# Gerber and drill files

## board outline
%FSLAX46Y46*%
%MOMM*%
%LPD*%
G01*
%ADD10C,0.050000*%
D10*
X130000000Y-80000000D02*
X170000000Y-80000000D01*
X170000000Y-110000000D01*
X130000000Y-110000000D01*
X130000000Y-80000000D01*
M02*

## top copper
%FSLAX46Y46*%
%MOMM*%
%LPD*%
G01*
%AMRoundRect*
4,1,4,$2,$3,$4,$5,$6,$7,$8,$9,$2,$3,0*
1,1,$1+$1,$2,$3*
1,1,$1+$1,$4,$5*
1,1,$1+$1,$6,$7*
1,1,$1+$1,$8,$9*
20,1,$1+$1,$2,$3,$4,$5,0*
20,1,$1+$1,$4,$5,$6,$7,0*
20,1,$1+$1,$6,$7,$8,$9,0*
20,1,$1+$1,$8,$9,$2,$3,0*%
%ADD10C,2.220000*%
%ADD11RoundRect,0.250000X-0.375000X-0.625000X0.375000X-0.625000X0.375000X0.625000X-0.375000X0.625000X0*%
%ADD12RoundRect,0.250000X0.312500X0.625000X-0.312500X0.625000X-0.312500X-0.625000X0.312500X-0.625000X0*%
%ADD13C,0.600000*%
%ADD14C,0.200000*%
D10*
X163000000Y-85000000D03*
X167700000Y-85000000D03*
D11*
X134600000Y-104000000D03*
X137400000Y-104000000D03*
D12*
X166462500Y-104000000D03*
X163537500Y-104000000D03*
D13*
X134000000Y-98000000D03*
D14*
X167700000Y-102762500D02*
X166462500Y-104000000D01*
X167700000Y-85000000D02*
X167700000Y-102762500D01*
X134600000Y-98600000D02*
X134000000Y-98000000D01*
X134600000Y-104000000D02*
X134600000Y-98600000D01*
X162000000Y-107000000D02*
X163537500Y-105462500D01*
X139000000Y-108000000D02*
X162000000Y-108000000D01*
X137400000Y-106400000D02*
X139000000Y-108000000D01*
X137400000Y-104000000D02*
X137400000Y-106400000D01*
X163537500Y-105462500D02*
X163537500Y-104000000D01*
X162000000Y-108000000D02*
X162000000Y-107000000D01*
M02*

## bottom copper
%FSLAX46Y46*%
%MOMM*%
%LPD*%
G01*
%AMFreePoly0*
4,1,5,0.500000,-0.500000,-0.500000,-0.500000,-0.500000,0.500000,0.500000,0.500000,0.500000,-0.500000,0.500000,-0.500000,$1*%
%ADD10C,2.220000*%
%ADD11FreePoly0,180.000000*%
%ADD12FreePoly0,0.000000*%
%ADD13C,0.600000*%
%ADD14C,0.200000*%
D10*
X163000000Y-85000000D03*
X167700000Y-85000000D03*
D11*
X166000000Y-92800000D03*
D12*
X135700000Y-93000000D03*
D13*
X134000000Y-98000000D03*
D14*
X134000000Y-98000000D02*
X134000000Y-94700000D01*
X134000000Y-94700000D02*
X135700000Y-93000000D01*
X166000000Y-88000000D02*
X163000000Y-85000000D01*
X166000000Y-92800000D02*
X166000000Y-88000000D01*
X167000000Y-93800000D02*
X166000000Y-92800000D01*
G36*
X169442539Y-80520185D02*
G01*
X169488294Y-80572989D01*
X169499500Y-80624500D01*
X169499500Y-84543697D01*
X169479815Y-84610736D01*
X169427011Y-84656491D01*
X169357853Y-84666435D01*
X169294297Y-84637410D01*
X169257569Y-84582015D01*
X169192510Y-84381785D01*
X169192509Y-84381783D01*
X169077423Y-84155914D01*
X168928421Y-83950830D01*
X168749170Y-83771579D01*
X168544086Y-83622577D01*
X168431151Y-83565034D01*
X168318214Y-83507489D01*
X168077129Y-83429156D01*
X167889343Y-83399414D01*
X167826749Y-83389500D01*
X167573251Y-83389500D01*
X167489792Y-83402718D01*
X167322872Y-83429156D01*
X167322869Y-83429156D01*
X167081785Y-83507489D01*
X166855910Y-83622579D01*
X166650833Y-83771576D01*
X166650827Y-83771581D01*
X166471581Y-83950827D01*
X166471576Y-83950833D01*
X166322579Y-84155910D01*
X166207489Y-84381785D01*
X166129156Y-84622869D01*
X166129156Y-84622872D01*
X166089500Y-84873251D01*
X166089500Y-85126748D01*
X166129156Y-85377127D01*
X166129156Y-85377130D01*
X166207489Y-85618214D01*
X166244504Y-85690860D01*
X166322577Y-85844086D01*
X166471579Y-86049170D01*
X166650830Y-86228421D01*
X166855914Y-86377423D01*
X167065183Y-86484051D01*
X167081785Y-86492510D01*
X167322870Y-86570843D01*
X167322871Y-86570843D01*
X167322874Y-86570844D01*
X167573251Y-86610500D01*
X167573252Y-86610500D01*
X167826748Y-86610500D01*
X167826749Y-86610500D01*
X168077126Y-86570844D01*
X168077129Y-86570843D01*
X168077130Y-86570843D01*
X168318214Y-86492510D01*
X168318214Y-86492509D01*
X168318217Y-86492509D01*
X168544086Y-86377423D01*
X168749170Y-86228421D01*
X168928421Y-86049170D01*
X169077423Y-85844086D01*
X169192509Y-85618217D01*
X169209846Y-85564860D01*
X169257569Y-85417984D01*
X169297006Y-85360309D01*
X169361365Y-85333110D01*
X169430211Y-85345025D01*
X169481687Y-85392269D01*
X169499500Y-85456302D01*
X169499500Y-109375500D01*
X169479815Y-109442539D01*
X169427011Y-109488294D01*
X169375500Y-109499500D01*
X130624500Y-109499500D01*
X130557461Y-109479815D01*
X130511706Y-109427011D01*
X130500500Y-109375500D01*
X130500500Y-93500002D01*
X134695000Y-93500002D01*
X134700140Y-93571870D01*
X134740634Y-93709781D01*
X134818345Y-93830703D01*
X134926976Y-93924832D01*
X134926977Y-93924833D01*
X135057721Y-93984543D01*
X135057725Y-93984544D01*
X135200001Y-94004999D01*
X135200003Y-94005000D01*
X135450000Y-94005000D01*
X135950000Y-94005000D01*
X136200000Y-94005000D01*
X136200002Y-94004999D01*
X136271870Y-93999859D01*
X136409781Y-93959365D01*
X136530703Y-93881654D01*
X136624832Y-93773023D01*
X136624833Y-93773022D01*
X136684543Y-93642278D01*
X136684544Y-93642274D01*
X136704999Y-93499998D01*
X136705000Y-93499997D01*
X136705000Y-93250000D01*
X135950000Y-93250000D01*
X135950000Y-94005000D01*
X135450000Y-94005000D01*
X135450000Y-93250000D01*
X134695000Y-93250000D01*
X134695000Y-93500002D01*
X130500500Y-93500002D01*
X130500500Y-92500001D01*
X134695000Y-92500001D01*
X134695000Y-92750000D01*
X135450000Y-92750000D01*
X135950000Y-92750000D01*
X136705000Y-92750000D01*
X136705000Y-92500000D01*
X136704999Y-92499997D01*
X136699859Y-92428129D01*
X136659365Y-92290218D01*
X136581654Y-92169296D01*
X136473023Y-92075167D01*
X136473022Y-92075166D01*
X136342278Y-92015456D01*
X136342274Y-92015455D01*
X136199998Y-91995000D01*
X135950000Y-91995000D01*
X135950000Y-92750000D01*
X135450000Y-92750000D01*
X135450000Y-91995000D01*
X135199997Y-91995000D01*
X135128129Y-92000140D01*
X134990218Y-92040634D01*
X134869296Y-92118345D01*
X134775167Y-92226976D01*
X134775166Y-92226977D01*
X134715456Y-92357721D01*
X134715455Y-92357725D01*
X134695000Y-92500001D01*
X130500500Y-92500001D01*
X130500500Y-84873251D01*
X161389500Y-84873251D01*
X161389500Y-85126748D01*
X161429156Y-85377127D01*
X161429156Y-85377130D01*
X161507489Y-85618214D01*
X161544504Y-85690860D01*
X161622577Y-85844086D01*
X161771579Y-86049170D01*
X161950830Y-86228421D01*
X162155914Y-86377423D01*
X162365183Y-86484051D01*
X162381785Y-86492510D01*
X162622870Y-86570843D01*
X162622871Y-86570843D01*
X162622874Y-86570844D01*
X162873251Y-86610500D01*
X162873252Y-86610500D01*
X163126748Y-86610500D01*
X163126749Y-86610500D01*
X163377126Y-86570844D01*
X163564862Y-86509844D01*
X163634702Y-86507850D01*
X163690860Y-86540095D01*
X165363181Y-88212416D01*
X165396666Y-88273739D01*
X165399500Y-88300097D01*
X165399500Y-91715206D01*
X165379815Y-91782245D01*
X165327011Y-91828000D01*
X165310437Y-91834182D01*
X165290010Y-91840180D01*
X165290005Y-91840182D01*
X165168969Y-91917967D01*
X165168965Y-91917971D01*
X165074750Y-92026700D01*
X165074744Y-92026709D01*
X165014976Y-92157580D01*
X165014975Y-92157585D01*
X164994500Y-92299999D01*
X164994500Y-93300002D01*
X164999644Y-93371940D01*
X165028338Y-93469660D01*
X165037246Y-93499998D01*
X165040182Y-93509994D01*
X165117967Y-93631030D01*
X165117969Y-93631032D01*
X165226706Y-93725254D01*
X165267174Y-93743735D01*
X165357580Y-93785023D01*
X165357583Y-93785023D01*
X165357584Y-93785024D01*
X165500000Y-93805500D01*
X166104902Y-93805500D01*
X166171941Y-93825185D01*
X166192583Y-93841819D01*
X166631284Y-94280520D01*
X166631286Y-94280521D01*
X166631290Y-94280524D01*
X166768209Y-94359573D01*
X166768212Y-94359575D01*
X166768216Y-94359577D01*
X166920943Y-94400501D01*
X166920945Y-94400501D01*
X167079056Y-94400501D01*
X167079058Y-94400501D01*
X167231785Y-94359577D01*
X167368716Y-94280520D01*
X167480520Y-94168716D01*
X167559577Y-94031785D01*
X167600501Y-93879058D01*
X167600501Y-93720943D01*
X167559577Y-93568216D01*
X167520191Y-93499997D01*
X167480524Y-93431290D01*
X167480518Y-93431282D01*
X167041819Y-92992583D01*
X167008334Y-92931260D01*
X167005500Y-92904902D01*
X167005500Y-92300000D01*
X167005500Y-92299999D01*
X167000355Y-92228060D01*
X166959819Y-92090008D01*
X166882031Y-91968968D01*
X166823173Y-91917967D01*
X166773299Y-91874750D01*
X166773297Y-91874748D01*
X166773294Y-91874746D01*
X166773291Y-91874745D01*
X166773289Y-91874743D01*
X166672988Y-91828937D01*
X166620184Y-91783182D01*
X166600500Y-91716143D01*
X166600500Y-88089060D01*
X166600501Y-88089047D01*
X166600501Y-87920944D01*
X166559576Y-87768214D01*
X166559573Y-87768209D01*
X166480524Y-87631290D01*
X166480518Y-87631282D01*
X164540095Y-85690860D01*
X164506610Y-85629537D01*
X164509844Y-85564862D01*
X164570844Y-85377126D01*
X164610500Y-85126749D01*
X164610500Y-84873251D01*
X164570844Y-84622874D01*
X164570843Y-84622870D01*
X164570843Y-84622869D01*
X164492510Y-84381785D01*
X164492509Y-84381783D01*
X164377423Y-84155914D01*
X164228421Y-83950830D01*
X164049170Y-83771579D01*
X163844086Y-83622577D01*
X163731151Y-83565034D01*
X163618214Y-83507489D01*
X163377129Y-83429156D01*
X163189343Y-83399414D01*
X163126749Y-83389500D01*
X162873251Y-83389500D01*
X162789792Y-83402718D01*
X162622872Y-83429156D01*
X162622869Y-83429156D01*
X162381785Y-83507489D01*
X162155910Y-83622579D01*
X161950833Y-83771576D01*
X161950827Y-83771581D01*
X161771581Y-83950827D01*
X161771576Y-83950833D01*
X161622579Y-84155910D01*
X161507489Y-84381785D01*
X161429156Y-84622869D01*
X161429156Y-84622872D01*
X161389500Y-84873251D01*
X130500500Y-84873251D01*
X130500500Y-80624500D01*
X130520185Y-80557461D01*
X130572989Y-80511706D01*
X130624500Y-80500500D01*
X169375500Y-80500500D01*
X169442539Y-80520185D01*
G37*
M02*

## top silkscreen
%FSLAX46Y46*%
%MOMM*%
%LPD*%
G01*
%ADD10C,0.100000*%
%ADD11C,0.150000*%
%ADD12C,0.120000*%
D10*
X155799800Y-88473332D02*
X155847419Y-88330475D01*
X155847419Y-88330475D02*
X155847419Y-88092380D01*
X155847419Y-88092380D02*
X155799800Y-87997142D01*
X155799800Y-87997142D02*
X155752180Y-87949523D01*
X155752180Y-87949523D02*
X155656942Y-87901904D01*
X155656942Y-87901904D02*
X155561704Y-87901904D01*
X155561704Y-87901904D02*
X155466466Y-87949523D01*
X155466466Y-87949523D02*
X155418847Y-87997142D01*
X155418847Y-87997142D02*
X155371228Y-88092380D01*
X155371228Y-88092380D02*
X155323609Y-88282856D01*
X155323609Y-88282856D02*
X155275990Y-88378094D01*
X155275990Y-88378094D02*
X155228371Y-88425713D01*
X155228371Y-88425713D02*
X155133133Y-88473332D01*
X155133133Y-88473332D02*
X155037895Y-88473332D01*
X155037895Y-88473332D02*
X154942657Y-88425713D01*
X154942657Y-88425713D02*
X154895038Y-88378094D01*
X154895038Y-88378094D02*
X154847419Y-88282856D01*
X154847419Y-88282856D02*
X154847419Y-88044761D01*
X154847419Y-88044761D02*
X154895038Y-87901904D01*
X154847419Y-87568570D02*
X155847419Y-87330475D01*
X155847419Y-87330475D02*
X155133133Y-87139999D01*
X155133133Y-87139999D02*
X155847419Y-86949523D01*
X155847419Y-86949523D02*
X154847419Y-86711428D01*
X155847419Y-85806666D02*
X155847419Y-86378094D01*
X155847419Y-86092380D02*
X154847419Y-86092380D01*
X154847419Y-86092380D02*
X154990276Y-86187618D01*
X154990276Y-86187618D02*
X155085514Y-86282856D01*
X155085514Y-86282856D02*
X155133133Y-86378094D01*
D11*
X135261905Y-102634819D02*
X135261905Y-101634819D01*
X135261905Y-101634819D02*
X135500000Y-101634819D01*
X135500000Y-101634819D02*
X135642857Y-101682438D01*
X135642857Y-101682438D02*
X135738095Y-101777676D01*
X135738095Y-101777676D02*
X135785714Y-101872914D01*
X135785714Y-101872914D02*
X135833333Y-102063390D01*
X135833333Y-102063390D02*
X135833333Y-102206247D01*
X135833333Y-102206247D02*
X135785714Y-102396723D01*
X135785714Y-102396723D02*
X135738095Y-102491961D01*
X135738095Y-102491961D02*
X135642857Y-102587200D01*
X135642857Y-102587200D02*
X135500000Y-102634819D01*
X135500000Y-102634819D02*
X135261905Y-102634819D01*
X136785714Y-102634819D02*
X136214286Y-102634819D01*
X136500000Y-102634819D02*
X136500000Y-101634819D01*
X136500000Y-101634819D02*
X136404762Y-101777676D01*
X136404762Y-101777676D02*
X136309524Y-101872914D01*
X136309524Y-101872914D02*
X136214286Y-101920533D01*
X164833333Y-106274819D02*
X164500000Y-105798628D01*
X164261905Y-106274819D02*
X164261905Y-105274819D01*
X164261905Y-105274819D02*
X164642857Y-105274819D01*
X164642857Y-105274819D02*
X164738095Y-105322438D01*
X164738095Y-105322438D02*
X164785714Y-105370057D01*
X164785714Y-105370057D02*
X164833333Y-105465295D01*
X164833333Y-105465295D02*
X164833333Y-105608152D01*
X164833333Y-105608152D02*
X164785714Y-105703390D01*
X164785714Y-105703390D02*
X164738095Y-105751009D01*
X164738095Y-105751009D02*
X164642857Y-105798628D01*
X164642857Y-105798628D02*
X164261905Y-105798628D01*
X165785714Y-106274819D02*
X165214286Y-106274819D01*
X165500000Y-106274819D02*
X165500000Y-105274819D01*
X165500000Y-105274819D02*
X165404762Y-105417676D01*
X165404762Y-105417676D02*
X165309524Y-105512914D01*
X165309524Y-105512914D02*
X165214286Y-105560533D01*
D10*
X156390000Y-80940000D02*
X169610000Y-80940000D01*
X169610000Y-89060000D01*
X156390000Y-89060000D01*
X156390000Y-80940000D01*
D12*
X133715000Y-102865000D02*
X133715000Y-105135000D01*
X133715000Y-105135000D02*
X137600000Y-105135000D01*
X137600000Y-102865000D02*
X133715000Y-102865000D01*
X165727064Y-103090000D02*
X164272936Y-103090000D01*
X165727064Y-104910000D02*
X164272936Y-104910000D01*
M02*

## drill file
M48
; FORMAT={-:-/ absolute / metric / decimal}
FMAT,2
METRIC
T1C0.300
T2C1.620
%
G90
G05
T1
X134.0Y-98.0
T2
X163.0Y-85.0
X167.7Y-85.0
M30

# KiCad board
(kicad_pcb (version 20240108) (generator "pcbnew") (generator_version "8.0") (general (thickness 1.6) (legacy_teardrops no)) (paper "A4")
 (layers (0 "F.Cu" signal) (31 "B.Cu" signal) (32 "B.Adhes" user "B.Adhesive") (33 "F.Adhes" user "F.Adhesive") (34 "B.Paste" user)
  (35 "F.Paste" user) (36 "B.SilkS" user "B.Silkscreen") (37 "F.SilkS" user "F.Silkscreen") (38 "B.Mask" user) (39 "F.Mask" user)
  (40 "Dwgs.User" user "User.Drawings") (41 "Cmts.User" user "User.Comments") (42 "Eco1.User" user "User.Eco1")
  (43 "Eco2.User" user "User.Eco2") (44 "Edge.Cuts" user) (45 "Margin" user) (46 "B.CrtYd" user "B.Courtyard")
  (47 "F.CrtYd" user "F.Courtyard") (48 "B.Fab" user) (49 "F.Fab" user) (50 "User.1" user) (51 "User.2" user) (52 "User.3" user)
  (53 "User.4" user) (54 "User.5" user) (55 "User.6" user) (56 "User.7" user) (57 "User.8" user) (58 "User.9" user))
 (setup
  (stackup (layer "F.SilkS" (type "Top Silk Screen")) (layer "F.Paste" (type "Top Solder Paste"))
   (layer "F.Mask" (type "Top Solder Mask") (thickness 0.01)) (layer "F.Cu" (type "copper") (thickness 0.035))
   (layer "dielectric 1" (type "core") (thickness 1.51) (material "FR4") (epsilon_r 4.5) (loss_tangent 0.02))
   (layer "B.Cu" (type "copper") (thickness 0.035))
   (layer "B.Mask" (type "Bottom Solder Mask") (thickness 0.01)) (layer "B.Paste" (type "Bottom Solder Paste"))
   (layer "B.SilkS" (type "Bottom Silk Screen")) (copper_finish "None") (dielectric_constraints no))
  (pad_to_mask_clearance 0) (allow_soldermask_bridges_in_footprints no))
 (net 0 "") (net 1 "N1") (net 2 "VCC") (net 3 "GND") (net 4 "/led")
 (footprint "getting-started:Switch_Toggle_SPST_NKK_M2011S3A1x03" (layer "F.Cu") (at 158.3 85 90)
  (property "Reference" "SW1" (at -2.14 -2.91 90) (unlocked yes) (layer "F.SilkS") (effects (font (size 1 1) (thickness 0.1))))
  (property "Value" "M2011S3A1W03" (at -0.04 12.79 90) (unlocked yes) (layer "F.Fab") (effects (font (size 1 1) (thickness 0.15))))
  (fp_rect (start -4.06 -1.91) (end 4.06 11.31) (stroke (width 0.1) (type default)) (fill none) (layer "F.SilkS"))
  (pad "2" thru_hole circle (at 0 4.7 90) (size 2.22 2.22) (drill 1.62) (layers "*.Cu" "*.Mask") (remove_unused_layers no) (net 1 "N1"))
  (pad "3" thru_hole circle (at 0 9.4 90) (size 2.22 2.22) (drill 1.62) (layers "*.Cu" "*.Mask") (remove_unused_layers no) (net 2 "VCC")))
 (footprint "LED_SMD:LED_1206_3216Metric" (layer "F.Cu") (at 136 104)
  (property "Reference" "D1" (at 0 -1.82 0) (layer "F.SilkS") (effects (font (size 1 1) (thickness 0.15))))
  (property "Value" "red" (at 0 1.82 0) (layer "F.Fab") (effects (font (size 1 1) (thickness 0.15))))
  (fp_line (start -2.285 -1.135) (end -2.285 1.135) (stroke (width 0.12) (type solid)) (layer "F.SilkS"))
  (fp_line (start -2.285 1.135) (end 1.6 1.135) (stroke (width 0.12) (type solid)) (layer "F.SilkS"))
  (fp_line (start 1.6 -1.135) (end -2.285 -1.135) (stroke (width 0.12) (type solid)) (layer "F.SilkS"))
  (pad "1" smd roundrect (at -1.4 0) (size 1.25 1.75) (layers "F.Cu" "F.Paste" "F.Mask") (roundrect_rratio 0.2) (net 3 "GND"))
  (pad "2" smd roundrect (at 1.4 0) (size 1.25 1.75) (layers "F.Cu" "F.Paste" "F.Mask") (roundrect_rratio 0.2) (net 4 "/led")))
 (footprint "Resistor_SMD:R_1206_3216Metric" (layer "F.Cu") (at 165 104 180)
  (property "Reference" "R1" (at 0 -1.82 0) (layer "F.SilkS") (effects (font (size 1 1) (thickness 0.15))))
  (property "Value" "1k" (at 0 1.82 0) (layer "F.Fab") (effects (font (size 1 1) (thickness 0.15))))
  (fp_line (start -0.727064 0.91) (end 0.727064 0.91) (stroke (width 0.12) (type solid)) (layer "F.SilkS"))
  (fp_line (start -0.727064 -0.91) (end 0.727064 -0.91) (stroke (width 0.12) (type solid)) (layer "F.SilkS"))
  (pad "1" smd roundrect (at -1.4625 0 180) (size 1.125 1.75) (layers "F.Cu" "F.Paste" "F.Mask") (roundrect_rratio 0.222222) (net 2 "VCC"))
  (pad "2" smd roundrect (at 1.4625 0 180) (size 1.125 1.75) (layers "F.Cu" "F.Paste" "F.Mask") (roundrect_rratio 0.222222) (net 4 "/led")))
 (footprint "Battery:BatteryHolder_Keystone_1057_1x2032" (layer "B.Cu") (at 150.85 92.9 180)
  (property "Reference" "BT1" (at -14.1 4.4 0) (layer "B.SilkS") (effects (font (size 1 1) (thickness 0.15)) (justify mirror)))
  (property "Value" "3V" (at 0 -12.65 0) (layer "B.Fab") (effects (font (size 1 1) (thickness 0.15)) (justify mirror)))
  (pad "1" smd custom (at -15.15 0.1 180) (size 1 1) (layers "B.Cu" "B.Paste" "B.Mask") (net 1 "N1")
   (options (clearance outline) (anchor rect)) (primitives))
  (pad "2" smd custom (at 15.15 -0.1) (size 1 1) (layers "B.Cu" "B.Paste" "B.Mask") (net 3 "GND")
   (options (clearance outline) (anchor rect)) (primitives)))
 (gr_rect (start 130 80) (end 170 110) (stroke (width 0.05) (type default)) (fill none) (layer "Edge.Cuts"))
 (segment (start 167.7 102.7625) (end 166.4625 104) (width 0.2) (layer "F.Cu") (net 2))
 (segment (start 167.7 85) (end 167.7 102.7625) (width 0.2) (layer "F.Cu") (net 2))
 (segment (start 134.6 98.6) (end 134 98) (width 0.2) (layer "F.Cu") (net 3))
 (segment (start 134.6 104) (end 134.6 98.6) (width 0.2) (layer "F.Cu") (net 3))
 (via (at 134 98) (size 0.6) (drill 0.3) (layers "F.Cu" "B.Cu") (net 3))
 (segment (start 134 98) (end 134 94.7) (width 0.2) (layer "B.Cu") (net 3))
 (segment (start 134 94.7) (end 135.7 93) (width 0.2) (layer "B.Cu") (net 3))
 (segment (start 162 107) (end 163.5375 105.4625) (width 0.2) (layer "F.Cu") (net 4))
 (segment (start 139 108) (end 162 108) (width 0.2) (layer "F.Cu") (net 4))
 (segment (start 137.4 106.4) (end 139 108) (width 0.2) (layer "F.Cu") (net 4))
 (segment (start 137.4 104) (end 137.4 106.4) (width 0.2) (layer "F.Cu") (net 4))
 (segment (start 163.5375 105.4625) (end 163.5375 104) (width 0.2) (layer "F.Cu") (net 4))
 (segment (start 162 108) (end 162 107) (width 0.2) (layer "F.Cu") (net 4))
 (segment (start 166 88) (end 163 85) (width 0.2) (layer "B.Cu") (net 1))
 (segment (start 166 92.8) (end 166 88) (width 0.2) (layer "B.Cu") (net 1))
 (segment (start 167 93.8) (end 166 92.8) (width 0.2) (layer "B.Cu") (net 1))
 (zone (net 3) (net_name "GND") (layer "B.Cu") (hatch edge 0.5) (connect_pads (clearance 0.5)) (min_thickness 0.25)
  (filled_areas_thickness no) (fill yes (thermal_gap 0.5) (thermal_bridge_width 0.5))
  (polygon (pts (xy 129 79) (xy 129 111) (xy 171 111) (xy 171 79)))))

